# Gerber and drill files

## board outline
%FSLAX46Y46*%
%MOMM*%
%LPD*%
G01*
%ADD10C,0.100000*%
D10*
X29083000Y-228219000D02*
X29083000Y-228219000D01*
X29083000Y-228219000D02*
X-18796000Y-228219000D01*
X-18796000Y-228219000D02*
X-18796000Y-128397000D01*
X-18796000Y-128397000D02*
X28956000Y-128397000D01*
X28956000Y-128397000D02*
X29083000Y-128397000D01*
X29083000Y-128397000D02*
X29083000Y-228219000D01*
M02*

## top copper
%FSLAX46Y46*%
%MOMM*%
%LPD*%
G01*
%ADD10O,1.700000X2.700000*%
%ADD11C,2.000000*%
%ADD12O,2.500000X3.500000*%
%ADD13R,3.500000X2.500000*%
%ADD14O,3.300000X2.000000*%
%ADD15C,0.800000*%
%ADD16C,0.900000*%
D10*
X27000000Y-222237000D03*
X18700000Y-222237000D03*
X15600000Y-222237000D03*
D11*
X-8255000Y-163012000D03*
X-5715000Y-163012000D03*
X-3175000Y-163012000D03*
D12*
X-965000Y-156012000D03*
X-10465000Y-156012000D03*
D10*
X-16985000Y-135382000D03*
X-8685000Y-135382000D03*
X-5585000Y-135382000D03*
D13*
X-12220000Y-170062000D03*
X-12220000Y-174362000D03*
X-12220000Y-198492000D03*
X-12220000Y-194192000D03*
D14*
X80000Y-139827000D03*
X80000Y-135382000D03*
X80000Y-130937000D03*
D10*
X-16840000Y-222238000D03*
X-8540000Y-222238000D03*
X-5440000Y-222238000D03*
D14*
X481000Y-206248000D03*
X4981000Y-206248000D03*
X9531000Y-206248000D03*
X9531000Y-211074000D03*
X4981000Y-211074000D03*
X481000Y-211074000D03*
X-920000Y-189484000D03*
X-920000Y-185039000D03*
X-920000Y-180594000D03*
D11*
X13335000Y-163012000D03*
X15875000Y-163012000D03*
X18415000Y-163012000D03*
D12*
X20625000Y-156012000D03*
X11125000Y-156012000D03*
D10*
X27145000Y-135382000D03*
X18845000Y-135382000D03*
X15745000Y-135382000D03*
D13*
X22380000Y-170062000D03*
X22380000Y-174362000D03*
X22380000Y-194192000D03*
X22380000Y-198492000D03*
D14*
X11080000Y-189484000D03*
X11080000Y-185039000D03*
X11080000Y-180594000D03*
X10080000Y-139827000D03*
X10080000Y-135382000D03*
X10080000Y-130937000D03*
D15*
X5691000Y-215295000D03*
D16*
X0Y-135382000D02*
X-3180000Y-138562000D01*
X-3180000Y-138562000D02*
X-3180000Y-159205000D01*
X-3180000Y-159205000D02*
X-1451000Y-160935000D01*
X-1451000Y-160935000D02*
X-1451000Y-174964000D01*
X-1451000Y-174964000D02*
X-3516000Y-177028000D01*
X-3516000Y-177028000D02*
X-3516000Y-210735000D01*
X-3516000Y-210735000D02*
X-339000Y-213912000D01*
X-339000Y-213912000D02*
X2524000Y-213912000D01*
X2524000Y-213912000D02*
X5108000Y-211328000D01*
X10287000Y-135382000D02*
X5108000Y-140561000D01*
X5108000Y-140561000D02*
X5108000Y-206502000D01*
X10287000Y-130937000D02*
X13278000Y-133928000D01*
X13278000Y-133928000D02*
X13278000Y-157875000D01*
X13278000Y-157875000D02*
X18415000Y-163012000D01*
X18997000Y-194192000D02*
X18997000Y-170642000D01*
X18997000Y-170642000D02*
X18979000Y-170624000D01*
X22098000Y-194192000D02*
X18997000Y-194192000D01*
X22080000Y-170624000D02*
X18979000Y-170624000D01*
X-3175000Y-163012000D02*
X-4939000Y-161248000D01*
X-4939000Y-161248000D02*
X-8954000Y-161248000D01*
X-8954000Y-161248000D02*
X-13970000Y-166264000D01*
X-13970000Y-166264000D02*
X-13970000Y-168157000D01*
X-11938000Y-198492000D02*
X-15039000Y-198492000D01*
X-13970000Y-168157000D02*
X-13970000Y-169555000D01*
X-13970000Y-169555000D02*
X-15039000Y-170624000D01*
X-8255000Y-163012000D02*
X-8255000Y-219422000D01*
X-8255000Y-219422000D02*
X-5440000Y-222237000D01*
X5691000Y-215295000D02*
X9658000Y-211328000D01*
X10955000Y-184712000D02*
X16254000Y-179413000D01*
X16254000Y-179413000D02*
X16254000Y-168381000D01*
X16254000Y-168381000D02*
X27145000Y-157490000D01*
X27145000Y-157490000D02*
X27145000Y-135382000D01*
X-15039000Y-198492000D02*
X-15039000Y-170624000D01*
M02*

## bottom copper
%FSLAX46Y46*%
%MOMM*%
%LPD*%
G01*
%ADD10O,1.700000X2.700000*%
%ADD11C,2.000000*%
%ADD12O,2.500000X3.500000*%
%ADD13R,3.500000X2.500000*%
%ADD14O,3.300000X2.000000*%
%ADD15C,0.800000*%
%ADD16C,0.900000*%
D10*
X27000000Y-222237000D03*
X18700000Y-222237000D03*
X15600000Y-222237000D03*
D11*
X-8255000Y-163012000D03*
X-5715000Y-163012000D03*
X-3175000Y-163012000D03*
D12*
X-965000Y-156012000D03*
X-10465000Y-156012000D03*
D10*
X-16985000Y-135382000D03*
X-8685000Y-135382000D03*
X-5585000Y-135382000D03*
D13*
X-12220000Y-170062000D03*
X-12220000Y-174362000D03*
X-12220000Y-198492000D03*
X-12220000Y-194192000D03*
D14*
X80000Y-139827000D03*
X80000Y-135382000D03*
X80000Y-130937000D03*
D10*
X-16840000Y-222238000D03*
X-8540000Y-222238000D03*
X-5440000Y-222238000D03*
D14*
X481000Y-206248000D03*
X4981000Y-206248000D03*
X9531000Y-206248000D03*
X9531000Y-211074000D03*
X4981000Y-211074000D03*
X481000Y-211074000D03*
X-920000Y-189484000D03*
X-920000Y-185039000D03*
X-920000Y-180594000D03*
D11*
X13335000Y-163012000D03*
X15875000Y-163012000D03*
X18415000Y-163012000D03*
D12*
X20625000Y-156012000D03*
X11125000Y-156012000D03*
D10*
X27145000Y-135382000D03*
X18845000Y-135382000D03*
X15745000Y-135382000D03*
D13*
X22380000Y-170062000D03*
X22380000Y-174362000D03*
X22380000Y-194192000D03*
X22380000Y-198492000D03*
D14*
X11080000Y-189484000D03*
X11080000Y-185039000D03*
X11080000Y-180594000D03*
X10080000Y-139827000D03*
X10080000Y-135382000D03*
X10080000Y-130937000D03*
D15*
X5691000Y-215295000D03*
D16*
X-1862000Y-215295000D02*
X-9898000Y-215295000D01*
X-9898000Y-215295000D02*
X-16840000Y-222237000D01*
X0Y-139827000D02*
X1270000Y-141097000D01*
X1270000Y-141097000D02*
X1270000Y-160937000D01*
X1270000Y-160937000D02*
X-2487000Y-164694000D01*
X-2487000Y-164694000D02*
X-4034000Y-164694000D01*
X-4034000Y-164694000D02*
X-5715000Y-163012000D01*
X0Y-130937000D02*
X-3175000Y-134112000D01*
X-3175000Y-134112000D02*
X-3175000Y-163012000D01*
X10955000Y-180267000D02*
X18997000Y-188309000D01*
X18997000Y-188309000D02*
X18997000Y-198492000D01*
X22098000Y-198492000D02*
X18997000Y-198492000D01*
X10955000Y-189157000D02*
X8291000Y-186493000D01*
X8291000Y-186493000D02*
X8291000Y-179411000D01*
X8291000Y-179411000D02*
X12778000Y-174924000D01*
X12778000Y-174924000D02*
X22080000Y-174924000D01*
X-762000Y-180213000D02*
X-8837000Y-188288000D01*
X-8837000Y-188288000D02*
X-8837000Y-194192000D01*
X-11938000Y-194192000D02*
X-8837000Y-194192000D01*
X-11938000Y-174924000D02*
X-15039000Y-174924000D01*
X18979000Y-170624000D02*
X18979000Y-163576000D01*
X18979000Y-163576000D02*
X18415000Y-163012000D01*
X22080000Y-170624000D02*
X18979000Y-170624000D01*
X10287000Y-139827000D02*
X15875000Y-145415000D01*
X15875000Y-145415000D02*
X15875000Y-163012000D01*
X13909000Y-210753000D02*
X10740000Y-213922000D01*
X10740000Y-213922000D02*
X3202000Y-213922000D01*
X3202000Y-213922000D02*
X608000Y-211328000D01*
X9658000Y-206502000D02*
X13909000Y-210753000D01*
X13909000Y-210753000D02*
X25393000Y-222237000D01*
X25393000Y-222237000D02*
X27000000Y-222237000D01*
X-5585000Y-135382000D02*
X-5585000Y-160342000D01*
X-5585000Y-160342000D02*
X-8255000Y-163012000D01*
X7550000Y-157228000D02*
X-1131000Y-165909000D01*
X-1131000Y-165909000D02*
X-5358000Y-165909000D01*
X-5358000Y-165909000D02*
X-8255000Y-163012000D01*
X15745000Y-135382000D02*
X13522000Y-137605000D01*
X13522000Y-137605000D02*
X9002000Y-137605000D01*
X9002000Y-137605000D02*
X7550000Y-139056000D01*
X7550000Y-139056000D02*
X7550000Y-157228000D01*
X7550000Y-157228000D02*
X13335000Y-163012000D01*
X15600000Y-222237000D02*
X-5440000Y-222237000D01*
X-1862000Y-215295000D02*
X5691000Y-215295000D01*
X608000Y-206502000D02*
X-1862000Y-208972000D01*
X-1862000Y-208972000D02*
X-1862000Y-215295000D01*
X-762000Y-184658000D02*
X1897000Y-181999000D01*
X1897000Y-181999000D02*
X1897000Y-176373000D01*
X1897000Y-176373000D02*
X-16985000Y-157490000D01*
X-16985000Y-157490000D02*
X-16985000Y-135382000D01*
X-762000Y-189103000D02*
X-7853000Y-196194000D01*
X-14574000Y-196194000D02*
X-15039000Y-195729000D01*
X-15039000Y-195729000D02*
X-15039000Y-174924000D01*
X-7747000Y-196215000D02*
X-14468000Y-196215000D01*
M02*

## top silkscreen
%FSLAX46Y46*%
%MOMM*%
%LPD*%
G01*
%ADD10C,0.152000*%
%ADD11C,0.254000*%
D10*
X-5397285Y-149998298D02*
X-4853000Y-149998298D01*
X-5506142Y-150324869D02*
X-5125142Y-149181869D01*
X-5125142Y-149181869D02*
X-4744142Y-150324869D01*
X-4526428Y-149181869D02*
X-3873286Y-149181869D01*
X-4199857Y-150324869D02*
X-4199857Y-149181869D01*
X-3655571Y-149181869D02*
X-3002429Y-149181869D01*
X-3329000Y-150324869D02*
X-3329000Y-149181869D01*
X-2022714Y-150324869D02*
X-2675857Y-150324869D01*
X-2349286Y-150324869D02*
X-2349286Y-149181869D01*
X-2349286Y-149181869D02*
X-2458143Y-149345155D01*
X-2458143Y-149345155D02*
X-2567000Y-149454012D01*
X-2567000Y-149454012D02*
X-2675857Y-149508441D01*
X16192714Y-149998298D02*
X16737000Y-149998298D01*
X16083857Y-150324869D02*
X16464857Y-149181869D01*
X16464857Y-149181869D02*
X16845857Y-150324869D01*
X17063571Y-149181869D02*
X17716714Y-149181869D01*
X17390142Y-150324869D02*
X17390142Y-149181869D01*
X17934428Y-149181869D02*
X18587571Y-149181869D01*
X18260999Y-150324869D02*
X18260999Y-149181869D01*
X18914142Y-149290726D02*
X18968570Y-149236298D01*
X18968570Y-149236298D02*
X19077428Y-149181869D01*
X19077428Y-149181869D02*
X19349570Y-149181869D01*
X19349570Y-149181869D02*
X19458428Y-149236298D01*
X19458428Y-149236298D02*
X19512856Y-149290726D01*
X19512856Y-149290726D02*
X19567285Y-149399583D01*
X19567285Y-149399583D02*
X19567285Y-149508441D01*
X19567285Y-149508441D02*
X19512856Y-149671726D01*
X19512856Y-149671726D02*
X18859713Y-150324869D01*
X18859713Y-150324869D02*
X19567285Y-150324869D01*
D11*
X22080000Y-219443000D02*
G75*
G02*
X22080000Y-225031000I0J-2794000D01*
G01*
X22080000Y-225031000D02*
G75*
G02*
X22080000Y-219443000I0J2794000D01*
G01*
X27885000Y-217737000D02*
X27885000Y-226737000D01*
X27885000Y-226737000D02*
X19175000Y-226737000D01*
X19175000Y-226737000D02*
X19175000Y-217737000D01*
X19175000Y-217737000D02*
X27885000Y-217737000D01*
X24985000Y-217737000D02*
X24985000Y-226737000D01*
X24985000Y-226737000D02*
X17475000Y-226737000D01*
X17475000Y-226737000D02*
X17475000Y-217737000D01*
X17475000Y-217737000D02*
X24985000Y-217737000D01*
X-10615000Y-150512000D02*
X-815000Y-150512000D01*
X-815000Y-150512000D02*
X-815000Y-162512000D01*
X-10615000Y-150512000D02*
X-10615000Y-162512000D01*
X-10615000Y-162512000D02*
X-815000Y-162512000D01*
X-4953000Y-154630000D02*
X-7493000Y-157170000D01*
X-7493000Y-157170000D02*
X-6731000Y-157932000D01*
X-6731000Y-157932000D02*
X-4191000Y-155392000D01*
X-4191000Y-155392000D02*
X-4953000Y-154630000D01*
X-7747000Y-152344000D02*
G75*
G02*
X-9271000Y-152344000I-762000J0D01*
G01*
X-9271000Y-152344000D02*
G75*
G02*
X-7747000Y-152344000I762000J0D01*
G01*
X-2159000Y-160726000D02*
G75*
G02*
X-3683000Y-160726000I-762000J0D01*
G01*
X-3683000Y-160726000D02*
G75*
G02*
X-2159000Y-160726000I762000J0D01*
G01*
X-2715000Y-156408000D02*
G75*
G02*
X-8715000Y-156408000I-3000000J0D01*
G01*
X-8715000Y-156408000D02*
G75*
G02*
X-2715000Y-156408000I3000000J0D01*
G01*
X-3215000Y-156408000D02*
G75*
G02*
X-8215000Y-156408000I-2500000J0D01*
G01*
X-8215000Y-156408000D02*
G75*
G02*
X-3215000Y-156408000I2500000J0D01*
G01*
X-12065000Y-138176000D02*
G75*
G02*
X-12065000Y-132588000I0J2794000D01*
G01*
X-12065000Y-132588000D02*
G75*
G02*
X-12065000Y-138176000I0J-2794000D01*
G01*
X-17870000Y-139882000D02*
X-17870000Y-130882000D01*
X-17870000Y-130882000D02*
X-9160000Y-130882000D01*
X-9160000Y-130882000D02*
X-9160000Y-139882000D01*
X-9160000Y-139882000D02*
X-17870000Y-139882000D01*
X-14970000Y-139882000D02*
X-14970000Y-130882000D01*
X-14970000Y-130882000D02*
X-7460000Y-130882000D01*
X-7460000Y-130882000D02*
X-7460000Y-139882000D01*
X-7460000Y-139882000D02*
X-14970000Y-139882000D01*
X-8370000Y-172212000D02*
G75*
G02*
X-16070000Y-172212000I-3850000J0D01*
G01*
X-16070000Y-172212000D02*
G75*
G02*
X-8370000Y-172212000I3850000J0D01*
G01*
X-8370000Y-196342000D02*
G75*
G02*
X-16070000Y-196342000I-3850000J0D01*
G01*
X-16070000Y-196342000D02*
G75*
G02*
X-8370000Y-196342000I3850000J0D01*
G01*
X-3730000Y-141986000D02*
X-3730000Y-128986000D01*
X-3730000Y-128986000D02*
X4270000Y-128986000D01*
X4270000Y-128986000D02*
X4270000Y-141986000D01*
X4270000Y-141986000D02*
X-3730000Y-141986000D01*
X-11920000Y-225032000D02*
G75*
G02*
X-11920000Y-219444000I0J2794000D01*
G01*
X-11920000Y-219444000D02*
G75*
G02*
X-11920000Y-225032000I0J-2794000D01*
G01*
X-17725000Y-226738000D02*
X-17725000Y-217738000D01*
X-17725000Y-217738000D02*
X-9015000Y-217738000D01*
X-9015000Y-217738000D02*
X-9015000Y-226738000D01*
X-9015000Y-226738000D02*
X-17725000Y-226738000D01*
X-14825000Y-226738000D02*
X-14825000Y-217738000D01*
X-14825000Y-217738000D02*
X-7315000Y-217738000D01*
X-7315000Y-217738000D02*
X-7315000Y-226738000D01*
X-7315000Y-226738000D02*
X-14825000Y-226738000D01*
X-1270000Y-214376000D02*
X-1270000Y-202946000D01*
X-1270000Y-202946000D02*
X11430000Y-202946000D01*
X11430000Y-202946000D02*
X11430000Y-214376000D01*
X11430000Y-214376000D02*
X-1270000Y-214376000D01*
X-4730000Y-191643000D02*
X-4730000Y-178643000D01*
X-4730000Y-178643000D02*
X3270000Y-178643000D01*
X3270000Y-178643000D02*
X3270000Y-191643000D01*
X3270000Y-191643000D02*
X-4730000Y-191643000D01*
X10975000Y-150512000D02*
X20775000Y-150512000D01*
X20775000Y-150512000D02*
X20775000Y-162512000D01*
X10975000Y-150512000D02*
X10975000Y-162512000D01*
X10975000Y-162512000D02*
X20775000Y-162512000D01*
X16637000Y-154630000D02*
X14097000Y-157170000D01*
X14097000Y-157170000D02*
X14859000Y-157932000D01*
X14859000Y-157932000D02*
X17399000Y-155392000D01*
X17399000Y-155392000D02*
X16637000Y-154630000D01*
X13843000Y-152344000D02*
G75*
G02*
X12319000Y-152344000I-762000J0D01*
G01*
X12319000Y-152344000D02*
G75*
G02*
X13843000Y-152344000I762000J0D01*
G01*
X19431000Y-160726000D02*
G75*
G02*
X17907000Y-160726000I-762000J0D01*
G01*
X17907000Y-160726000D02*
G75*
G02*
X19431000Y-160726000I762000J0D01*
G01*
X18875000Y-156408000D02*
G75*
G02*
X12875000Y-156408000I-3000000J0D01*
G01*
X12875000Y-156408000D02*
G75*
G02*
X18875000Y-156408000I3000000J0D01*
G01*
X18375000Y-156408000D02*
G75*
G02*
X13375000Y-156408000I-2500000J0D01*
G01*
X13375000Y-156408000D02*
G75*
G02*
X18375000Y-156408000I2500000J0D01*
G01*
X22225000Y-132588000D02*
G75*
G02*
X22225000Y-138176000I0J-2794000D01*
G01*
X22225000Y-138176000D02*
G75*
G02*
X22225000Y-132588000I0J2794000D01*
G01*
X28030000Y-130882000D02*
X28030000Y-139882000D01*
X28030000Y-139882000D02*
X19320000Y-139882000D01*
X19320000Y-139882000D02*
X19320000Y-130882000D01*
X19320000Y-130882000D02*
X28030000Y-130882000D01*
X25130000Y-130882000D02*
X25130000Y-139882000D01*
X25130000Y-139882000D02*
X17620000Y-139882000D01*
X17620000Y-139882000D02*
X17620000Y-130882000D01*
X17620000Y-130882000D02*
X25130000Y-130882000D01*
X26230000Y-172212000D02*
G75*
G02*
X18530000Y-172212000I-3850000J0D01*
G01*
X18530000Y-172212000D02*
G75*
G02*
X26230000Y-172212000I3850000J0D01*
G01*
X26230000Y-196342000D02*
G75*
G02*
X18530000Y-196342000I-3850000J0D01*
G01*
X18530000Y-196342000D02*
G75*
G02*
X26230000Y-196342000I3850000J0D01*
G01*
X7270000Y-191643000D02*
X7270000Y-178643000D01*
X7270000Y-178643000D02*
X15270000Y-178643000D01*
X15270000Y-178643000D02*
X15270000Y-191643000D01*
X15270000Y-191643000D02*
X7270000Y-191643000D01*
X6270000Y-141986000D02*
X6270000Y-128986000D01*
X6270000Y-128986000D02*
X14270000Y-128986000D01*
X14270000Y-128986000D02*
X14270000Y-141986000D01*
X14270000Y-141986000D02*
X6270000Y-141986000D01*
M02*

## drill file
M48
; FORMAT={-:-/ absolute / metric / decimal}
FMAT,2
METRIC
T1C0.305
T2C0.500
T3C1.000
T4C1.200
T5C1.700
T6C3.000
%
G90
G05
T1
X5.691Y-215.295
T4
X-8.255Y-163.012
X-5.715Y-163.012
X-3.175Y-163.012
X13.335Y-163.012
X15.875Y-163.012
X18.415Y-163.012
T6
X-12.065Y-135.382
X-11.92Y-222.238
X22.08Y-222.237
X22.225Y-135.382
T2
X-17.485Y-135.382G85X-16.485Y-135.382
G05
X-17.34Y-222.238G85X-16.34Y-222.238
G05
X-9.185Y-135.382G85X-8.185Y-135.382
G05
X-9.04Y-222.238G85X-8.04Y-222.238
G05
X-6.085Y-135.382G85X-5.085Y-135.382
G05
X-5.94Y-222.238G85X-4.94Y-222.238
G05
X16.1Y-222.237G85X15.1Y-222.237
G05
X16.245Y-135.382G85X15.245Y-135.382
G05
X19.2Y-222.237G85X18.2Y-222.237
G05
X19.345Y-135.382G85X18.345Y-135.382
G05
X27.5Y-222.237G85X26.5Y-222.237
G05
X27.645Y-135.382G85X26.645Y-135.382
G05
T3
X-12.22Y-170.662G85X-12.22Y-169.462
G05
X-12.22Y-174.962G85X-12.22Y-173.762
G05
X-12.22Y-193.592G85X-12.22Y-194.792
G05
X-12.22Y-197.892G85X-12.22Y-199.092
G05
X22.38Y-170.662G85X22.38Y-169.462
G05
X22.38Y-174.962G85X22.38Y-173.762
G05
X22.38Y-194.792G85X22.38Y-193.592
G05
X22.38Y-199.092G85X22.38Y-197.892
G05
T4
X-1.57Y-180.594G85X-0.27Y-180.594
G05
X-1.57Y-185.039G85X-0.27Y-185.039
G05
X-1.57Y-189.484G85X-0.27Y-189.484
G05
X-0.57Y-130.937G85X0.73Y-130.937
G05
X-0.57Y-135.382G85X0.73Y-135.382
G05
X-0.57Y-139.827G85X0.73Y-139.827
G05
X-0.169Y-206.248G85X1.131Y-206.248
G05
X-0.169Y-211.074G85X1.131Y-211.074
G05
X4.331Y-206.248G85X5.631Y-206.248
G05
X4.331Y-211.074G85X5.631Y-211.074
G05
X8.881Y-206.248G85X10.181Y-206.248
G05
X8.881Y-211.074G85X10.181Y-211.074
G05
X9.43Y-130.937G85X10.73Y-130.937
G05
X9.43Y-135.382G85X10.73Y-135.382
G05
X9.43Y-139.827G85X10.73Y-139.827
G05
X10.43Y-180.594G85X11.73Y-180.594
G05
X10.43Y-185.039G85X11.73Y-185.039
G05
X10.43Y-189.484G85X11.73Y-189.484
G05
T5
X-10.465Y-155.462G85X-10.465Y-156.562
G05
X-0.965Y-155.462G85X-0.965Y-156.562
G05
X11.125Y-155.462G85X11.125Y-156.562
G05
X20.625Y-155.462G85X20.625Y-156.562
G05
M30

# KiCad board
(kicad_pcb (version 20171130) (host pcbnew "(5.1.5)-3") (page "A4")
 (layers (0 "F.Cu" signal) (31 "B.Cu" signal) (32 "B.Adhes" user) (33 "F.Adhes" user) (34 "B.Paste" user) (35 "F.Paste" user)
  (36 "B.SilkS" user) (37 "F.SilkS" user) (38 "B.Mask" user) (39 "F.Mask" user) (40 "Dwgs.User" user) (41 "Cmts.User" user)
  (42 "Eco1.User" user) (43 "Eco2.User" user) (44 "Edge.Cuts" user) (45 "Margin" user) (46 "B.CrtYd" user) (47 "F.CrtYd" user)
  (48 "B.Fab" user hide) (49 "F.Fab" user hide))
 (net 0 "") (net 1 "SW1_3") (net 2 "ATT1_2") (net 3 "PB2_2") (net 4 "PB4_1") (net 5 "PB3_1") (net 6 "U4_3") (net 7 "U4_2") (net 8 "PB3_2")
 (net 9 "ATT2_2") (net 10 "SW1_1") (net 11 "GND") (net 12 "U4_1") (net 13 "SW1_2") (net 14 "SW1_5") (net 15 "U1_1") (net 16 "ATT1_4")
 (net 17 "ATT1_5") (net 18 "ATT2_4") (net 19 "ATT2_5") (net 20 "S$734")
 (segment (start -1.862 215.295) (end -9.898 215.295) (width 0.9) (layer "B.Cu") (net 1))
 (segment (start -9.898 215.295) (end -16.84 222.237) (width 0.9) (layer "B.Cu") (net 1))
 (segment (start 0 139.827) (end 1.27 141.097) (width 0.9) (layer "B.Cu") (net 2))
 (segment (start 1.27 141.097) (end 1.27 160.937) (width 0.9) (layer "B.Cu") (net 2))
 (segment (start 1.27 160.937) (end -2.487 164.694) (width 0.9) (layer "B.Cu") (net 2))
 (segment (start -2.487 164.694) (end -4.034 164.694) (width 0.9) (layer "B.Cu") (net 2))
 (segment (start -4.034 164.694) (end -5.715 163.012) (width 0.9) (layer "B.Cu") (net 2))
 (segment (start 0 130.937) (end -3.175 134.112) (width 0.9) (layer "B.Cu") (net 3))
 (segment (start -3.175 134.112) (end -3.175 163.012) (width 0.9) (layer "B.Cu") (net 3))
 (segment (start 10.955 180.267) (end 18.997 188.309) (width 0.9) (layer "B.Cu") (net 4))
 (segment (start 18.997 188.309) (end 18.997 198.492) (width 0.9) (layer "B.Cu") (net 4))
 (segment (start 22.098 198.492) (end 18.997 198.492) (width 0.9) (layer "B.Cu") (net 4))
 (segment (start 10.955 189.157) (end 8.291 186.493) (width 0.9) (layer "B.Cu") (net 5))
 (segment (start 8.291 186.493) (end 8.291 179.411) (width 0.9) (layer "B.Cu") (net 5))
 (segment (start 8.291 179.411) (end 12.778 174.924) (width 0.9) (layer "B.Cu") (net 5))
 (segment (start 12.778 174.924) (end 22.08 174.924) (width 0.9) (layer "B.Cu") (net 5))
 (segment (start -0.762 180.213) (end -8.837 188.288) (width 0.9) (layer "B.Cu") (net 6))
 (segment (start -8.837 188.288) (end -8.837 194.192) (width 0.9) (layer "B.Cu") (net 6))
 (segment (start -11.938 194.192) (end -8.837 194.192) (width 0.9) (layer "B.Cu") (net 6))
 (segment (start -11.938 174.924) (end -15.039 174.924) (width 0.9) (layer "B.Cu") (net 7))
 (segment (start 18.979 170.624) (end 18.979 163.576) (width 0.9) (layer "B.Cu") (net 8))
 (segment (start 18.979 163.576) (end 18.415 163.012) (width 0.9) (layer "B.Cu") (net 8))
 (segment (start 22.08 170.624) (end 18.979 170.624) (width 0.9) (layer "B.Cu") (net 8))
 (segment (start 10.287 139.827) (end 15.875 145.415) (width 0.9) (layer "B.Cu") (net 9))
 (segment (start 15.875 145.415) (end 15.875 163.012) (width 0.9) (layer "B.Cu") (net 9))
 (segment (start 13.909 210.753) (end 10.74 213.922) (width 0.9) (layer "B.Cu") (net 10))
 (segment (start 10.74 213.922) (end 3.202 213.922) (width 0.9) (layer "B.Cu") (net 10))
 (segment (start 3.202 213.922) (end 0.608 211.328) (width 0.9) (layer "B.Cu") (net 10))
 (segment (start 9.658 206.502) (end 13.909 210.753) (width 0.9) (layer "B.Cu") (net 10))
 (segment (start 13.909 210.753) (end 25.393 222.237) (width 0.9) (layer "B.Cu") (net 10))
 (segment (start 25.393 222.237) (end 27 222.237) (width 0.9) (layer "B.Cu") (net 10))
 (segment (start -5.585 135.382) (end -5.585 160.342) (width 0.9) (layer "B.Cu") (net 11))
 (segment (start -5.585 160.342) (end -8.255 163.012) (width 0.9) (layer "B.Cu") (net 11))
 (segment (start 7.55 157.228) (end -1.131 165.909) (width 0.9) (layer "B.Cu") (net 11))
 (segment (start -1.131 165.909) (end -5.358 165.909) (width 0.9) (layer "B.Cu") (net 11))
 (segment (start -5.358 165.909) (end -8.255 163.012) (width 0.9) (layer "B.Cu") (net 11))
 (segment (start 15.745 135.382) (end 13.522 137.605) (width 0.9) (layer "B.Cu") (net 11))
 (segment (start 13.522 137.605) (end 9.002 137.605) (width 0.9) (layer "B.Cu") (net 11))
 (segment (start 9.002 137.605) (end 7.55 139.056) (width 0.9) (layer "B.Cu") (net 11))
 (segment (start 7.55 139.056) (end 7.55 157.228) (width 0.9) (layer "B.Cu") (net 11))
 (segment (start 7.55 157.228) (end 13.335 163.012) (width 0.9) (layer "B.Cu") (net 11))
 (segment (start 15.6 222.237) (end -5.44 222.237) (width 0.9) (layer "B.Cu") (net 11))
 (segment (start -1.862 215.295) (end 5.691 215.295) (width 0.9) (layer "B.Cu") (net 1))
 (segment (start 0.608 206.502) (end -1.862 208.972) (width 0.9) (layer "B.Cu") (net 1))
 (segment (start -1.862 208.972) (end -1.862 215.295) (width 0.9) (layer "B.Cu") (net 1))
 (segment (start -0.762 184.658) (end 1.897 181.999) (width 0.9) (layer "B.Cu") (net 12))
 (segment (start 1.897 181.999) (end 1.897 176.373) (width 0.9) (layer "B.Cu") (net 12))
 (segment (start 1.897 176.373) (end -16.985 157.49) (width 0.9) (layer "B.Cu") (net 12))
 (segment (start -16.985 157.49) (end -16.985 135.382) (width 0.9) (layer "B.Cu") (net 12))
 (segment (start -0.762 189.103) (end -7.853 196.194) (width 0.9) (layer "B.Cu") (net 7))
 (segment (start -14.574 196.194) (end -15.039 195.729) (width 0.9) (layer "B.Cu") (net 7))
 (segment (start -15.039 195.729) (end -15.039 174.924) (width 0.9) (layer "B.Cu") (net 7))
 (segment (start -7.747 196.215) (end -14.468 196.215) (width 0.9) (layer "B.Cu") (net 7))
 (gr_line (start 29.083 228.219) (end 29.083 228.219) (width 0.1) (layer "Edge.Cuts"))
 (gr_line (start 29.083 228.219) (end -18.796 228.219) (width 0.1) (layer "Edge.Cuts"))
 (gr_line (start -18.796 228.219) (end -18.796 128.397) (width 0.1) (layer "Edge.Cuts"))
 (gr_line (start -18.796 128.397) (end 28.956 128.397) (width 0.1) (layer "Edge.Cuts"))
 (gr_line (start 28.956 128.397) (end 29.083 128.397) (width 0.1) (layer "Edge.Cuts"))
 (gr_line (start 29.083 128.397) (end 29.083 228.219) (width 0.1) (layer "Edge.Cuts"))
 (segment (start 0 135.382) (end -3.18 138.562) (width 0.9) (layer "F.Cu") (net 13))
 (segment (start -3.18 138.562) (end -3.18 159.205) (width 0.9) (layer "F.Cu") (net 13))
 (segment (start -3.18 159.205) (end -1.451 160.935) (width 0.9) (layer "F.Cu") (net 13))
 (segment (start -1.451 160.935) (end -1.451 174.964) (width 0.9) (layer "F.Cu") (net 13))
 (segment (start -1.451 174.964) (end -3.516 177.028) (width 0.9) (layer "F.Cu") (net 13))
 (segment (start -3.516 177.028) (end -3.516 210.735) (width 0.9) (layer "F.Cu") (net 13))
 (segment (start -3.516 210.735) (end -0.339 213.912) (width 0.9) (layer "F.Cu") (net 13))
 (segment (start -0.339 213.912) (end 2.524 213.912) (width 0.9) (layer "F.Cu") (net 13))
 (segment (start 2.524 213.912) (end 5.108 211.328) (width 0.9) (layer "F.Cu") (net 13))
 (segment (start 10.287 135.382) (end 5.108 140.561) (width 0.9) (layer "F.Cu") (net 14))
 (segment (start 5.108 140.561) (end 5.108 206.502) (width 0.9) (layer "F.Cu") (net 14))
 (segment (start 10.287 130.937) (end 13.278 133.928) (width 0.9) (layer "F.Cu") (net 8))
 (segment (start 13.278 133.928) (end 13.278 157.875) (width 0.9) (layer "F.Cu") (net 8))
 (segment (start 13.278 157.875) (end 18.415 163.012) (width 0.9) (layer "F.Cu") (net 8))
 (segment (start 18.997 194.192) (end 18.997 170.642) (width 0.9) (layer "F.Cu") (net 8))
 (segment (start 18.997 170.642) (end 18.979 170.624) (width 0.9) (layer "F.Cu") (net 8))
 (segment (start 22.098 194.192) (end 18.997 194.192) (width 0.9) (layer "F.Cu") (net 8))
 (segment (start 22.08 170.624) (end 18.979 170.624) (width 0.9) (layer "F.Cu") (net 8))
 (segment (start -3.175 163.012) (end -4.939 161.248) (width 0.9) (layer "F.Cu") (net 3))
 (segment (start -4.939 161.248) (end -8.954 161.248) (width 0.9) (layer "F.Cu") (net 3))
 (segment (start -8.954 161.248) (end -13.97 166.264) (width 0.9) (layer "F.Cu") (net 3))
 (segment (start -13.97 166.264) (end -13.97 168.157) (width 0.9) (layer "F.Cu") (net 3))
 (segment (start -11.938 198.492) (end -15.039 198.492) (width 0.9) (layer "F.Cu") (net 3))
 (segment (start -13.97 168.157) (end -13.97 169.555) (width 0.9) (layer "F.Cu") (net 3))
 (segment (start -13.97 169.555) (end -15.039 170.624) (width 0.9) (layer "F.Cu") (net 3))
 (segment (start -8.255 163.012) (end -8.255 219.422) (width 0.9) (layer "F.Cu") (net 11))
 (segment (start -8.255 219.422) (end -5.44 222.237) (width 0.9) (layer "F.Cu") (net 11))
 (segment (start 5.691 215.295) (end 9.658 211.328) (width 0.9) (layer "F.Cu") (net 1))
 (segment (start 10.955 184.712) (end 16.254 179.413) (width 0.9) (layer "F.Cu") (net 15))
 (segment (start 16.254 179.413) (end 16.254 168.381) (width 0.9) (layer "F.Cu") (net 15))
 (segment (start 16.254 168.381) (end 27.145 157.49) (width 0.9) (layer "F.Cu") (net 15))
 (segment (start 27.145 157.49) (end 27.145 135.382) (width 0.9) (layer "F.Cu") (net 15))
 (segment (start -15.039 198.492) (end -15.039 170.624) (width 0.9) (layer "F.Cu") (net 3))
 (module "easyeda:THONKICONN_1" (layer "F.Cu") (at 22.08 222.237 -90)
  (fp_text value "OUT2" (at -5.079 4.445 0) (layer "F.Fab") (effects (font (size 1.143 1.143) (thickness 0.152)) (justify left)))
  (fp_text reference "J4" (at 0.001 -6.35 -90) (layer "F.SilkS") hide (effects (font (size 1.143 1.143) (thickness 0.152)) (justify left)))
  (fp_arc (start 0 0) (end -2.794 0) (angle 180) (width 0.254) (layer "F.SilkS"))
  (fp_arc (start 0 0) (end 2.794 0) (angle 180) (width 0.254) (layer "F.SilkS"))
  (fp_line (start -4.5 -5.805) (end 4.5 -5.805) (width 0.254) (layer "F.SilkS"))
  (fp_line (start 4.5 -5.805) (end 4.5 2.905) (width 0.254) (layer "F.SilkS"))
  (fp_line (start 4.5 2.905) (end -4.5 2.905) (width 0.254) (layer "F.SilkS"))
  (fp_line (start -4.5 2.905) (end -4.5 -5.805) (width 0.254) (layer "F.SilkS"))
  (fp_line (start -4.5 -2.905) (end 4.5 -2.905) (width 0.254) (layer "F.SilkS"))
  (fp_line (start 4.5 -2.905) (end 4.5 4.605) (width 0.254) (layer "F.SilkS"))
  (fp_line (start 4.5 4.605) (end -4.5 4.605) (width 0.254) (layer "F.SilkS"))
  (fp_line (start -4.5 4.605) (end -4.5 -2.905) (width 0.254) (layer "F.SilkS"))
  (pad "" np_thru_hole circle (at 0 0) (size 3 3) (drill 3) (layers "*.Cu" "*.Mask"))
  (pad 3 thru_hole oval (at 0 -4.92 -90) (size 2.7 1.7) (layers "*.Cu" "*.Paste" "*.Mask") (drill oval 0.5 1.5) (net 10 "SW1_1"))
  (pad 2 thru_hole oval (at 0 3.38 -90) (size 2.7 1.7) (layers "*.Cu" "*.Paste" "*.Mask") (drill oval 0.5 1.5))
  (pad 1 thru_hole oval (at 0 6.48 -90) (size 2.7 1.7) (layers "*.Cu" "*.Paste" "*.Mask") (drill oval 0.5 1.5) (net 11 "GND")))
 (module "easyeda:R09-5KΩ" (layer "F.Cu") (at -5.715 159.512)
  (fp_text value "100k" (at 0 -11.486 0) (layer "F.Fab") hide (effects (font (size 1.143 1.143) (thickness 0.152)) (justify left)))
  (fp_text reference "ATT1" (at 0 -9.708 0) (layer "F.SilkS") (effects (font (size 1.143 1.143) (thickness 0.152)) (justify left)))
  (fp_line (start -4.9 -9) (end 4.9 -9) (width 0.254) (layer "F.SilkS"))
  (fp_line (start 4.9 -9) (end 4.9 3) (width 0.254) (layer "F.SilkS"))
  (fp_line (start -4.9 -9) (end -4.9 3) (width 0.254) (layer "F.SilkS"))
  (fp_line (start -4.9 3) (end 4.9 3) (width 0.254) (layer "F.SilkS"))
  (fp_line (start 0.762 -4.882) (end -1.778 -2.342) (width 0.254) (layer "F.SilkS"))
  (fp_line (start -1.778 -2.342) (end -1.016 -1.58) (width 0.254) (layer "F.SilkS"))
  (fp_line (start -1.016 -1.58) (end 1.524 -4.12) (width 0.254) (layer "F.SilkS"))
  (fp_line (start 1.524 -4.12) (end 0.762 -4.882) (width 0.254) (layer "F.SilkS"))
  (fp_circle (center -2.794 -7.168) (end -2.032 -7.168) (layer "F.SilkS") (width 0.254))
  (fp_circle (center 2.794 1.214) (end 3.556 1.214) (layer "F.SilkS") (width 0.254))
  (fp_circle (center 0 -3.104) (end 3 -3.104) (layer "F.SilkS") (width 0.254))
  (fp_circle (center 0 -3.104) (end 2.5 -3.104) (layer "F.SilkS") (width 0.254))
  (pad 1 thru_hole circle (at -2.54 3.5 0) (size 2 2) (layers "*.Cu" "*.Paste" "*.Mask") (drill 1.2) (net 11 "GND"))
  (pad 2 thru_hole circle (at 0 3.5 0) (size 2 2) (layers "*.Cu" "*.Paste" "*.Mask") (drill 1.2) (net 2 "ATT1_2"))
  (pad 3 thru_hole circle (at 2.54 3.5 0) (size 2 2) (layers "*.Cu" "*.Paste" "*.Mask") (drill 1.2) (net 3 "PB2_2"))
  (pad 4 thru_hole oval (at 4.75 -3.5 0) (size 2.5 3.5) (layers "*.Cu" "*.Paste" "*.Mask") (drill oval 1.7 2.8) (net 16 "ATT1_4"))
  (pad 5 thru_hole oval (at -4.75 -3.5 0) (size 2.5 3.5) (layers "*.Cu" "*.Paste" "*.Mask") (drill oval 1.7 2.8) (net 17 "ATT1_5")))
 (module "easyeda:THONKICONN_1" (layer "F.Cu") (at -12.065 135.382 90)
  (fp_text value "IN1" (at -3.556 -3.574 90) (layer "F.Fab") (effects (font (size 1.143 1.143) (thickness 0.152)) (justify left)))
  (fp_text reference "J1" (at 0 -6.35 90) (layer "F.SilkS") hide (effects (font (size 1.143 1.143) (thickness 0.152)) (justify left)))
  (fp_arc (start 0 0) (end -2.794 0) (angle 180) (width 0.254) (layer "F.SilkS"))
  (fp_arc (start 0 0) (end 2.794 0) (angle 180) (width 0.254) (layer "F.SilkS"))
  (pad "" np_thru_hole circle (at 0 0) (size 3 3) (drill 3) (layers "*.Cu" "*.Mask"))
  (fp_line (start -4.5 -5.805) (end 4.5 -5.805) (width 0.254) (layer "F.SilkS"))
  (fp_line (start 4.5 -5.805) (end 4.5 2.905) (width 0.254) (layer "F.SilkS"))
  (fp_line (start 4.5 2.905) (end -4.5 2.905) (width 0.254) (layer "F.SilkS"))
  (fp_line (start -4.5 2.905) (end -4.5 -5.805) (width 0.254) (layer "F.SilkS"))
  (fp_line (start -4.5 -2.905) (end 4.5 -2.905) (width 0.254) (layer "F.SilkS"))
  (fp_line (start 4.5 -2.905) (end 4.5 4.605) (width 0.254) (layer "F.SilkS"))
  (fp_line (start 4.5 4.605) (end -4.5 4.605) (width 0.254) (layer "F.SilkS"))
  (fp_line (start -4.5 4.605) (end -4.5 -2.905) (width 0.254) (layer "F.SilkS"))
  (pad 3 thru_hole oval (at 0 -4.92 90) (size 2.7 1.7) (layers "*.Cu" "*.Paste" "*.Mask") (drill oval 0.5 1.5) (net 12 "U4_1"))
  (pad 2 thru_hole oval (at 0 3.38 90) (size 2.7 1.7) (layers "*.Cu" "*.Paste" "*.Mask") (drill oval 0.5 1.5))
  (pad 1 thru_hole oval (at 0 6.48 90) (size 2.7 1.7) (layers "*.Cu" "*.Paste" "*.Mask") (drill oval 0.5 1.5) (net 11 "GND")))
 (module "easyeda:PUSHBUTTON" (layer "F.Cu") (at -12.22 172.212 90)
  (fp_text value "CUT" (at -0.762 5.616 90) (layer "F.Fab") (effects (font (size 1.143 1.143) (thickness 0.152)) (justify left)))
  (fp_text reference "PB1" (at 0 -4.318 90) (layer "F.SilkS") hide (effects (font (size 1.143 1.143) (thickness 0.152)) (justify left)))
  (fp_circle (center 0 0) (end 3.85 0) (layer "F.SilkS") (width 0.254))
  (pad 2 thru_hole rect (at 2.15 0 180) (size 3.5 2.5) (layers "*.Cu" "*.Paste" "*.Mask") (drill oval 1 2.2) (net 3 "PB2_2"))
  (pad 1 thru_hole rect (at -2.15 0 180) (size 3.5 2.5) (layers "*.Cu" "*.Paste" "*.Mask") (drill oval 1 2.2) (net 7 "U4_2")))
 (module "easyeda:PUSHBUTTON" (layer "F.Cu") (at -12.22 196.342 -90)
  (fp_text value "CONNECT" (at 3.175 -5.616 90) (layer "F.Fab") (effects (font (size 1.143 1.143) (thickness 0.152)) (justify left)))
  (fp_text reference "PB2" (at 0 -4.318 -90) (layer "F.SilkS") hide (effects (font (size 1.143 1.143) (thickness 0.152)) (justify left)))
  (fp_circle (center 0 0) (end 3.85 0) (layer "F.SilkS") (width 0.254))
  (pad 2 thru_hole rect (at 2.15 0 0) (size 3.5 2.5) (layers "*.Cu" "*.Paste" "*.Mask") (drill oval 1 2.2) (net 3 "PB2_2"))
  (pad 1 thru_hole rect (at -2.15 0 0) (size 3.5 2.5) (layers "*.Cu" "*.Paste" "*.Mask") (drill oval 1 2.2) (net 6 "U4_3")))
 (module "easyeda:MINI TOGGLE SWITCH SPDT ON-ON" (layer "F.Cu") (at 0.08 135.382 90)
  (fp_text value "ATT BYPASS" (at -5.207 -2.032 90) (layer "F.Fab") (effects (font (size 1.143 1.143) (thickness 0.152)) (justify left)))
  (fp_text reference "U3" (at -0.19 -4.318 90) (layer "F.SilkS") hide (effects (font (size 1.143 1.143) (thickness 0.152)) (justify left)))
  (fp_line (start -6.604 -3.81) (end 6.396 -3.81) (width 0.254) (layer "F.SilkS") (status 40000))
  (fp_line (start 6.396 -3.81) (end 6.396 4.19) (width 0.254) (layer "F.SilkS") (status 40000))
  (fp_line (start 6.396 4.19) (end -6.604 4.19) (width 0.254) (layer "F.SilkS") (status 40000))
  (fp_line (start -6.604 4.19) (end -6.604 -3.81) (width 0.254) (layer "F.SilkS") (status 40000))
  (pad 2 thru_hole oval (at -4.445 0 90) (size 2 3.3) (layers "*.Cu" "*.Paste" "*.Mask") (drill oval 1.2 2.5) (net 2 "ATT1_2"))
  (pad 1 thru_hole oval (at 0 0 90) (size 2 3.3) (layers "*.Cu" "*.Paste" "*.Mask") (drill oval 1.2 2.5) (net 13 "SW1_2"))
  (pad 3 thru_hole oval (at 4.445 0 90) (size 2 3.3) (layers "*.Cu" "*.Paste" "*.Mask") (drill oval 1.2 2.5) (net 3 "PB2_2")))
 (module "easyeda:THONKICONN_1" (layer "F.Cu") (at -11.92 222.238 90)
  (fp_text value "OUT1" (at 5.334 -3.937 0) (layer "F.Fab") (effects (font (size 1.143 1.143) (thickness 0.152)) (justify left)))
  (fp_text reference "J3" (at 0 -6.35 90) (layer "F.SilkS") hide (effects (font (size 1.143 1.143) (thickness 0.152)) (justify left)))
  (fp_arc (start 0 0) (end -2.794 0) (angle 180) (width 0.254) (layer "F.SilkS"))
  (fp_arc (start 0 0) (end 2.794 0) (angle 180) (width 0.254) (layer "F.SilkS"))
  (fp_line (start -4.5 -5.805) (end 4.5 -5.805) (width 0.254) (layer "F.SilkS"))
  (fp_line (start 4.5 -5.805) (end 4.5 2.905) (width 0.254) (layer "F.SilkS"))
  (fp_line (start 4.5 2.905) (end -4.5 2.905) (width 0.254) (layer "F.SilkS"))
  (fp_line (start -4.5 2.905) (end -4.5 -5.805) (width 0.254) (layer "F.SilkS"))
  (fp_line (start -4.5 -2.905) (end 4.5 -2.905) (width 0.254) (layer "F.SilkS"))
  (fp_line (start 4.5 -2.905) (end 4.5 4.605) (width 0.254) (layer "F.SilkS"))
  (fp_line (start 4.5 4.605) (end -4.5 4.605) (width 0.254) (layer "F.SilkS"))
  (fp_line (start -4.5 4.605) (end -4.5 -2.905) (width 0.254) (layer "F.SilkS"))
  (pad "" np_thru_hole circle (at 0 0) (size 3 3) (drill 3) (layers "*.Cu" "*.Mask"))
  (pad 3 thru_hole oval (at 0 -4.92 90) (size 2.7 1.7) (layers "*.Cu" "*.Paste" "*.Mask") (drill oval 0.5 1.5) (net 1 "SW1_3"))
  (pad 2 thru_hole oval (at 0 3.38 90) (size 2.7 1.7) (layers "*.Cu" "*.Paste" "*.Mask") (drill oval 0.5 1.5))
  (pad 1 thru_hole oval (at 0 6.48 90) (size 2.7 1.7) (layers "*.Cu" "*.Paste" "*.Mask") (drill oval 0.5 1.5) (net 11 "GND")))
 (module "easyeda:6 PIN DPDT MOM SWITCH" (layer "F.Cu") (at 11.43 214.376 90)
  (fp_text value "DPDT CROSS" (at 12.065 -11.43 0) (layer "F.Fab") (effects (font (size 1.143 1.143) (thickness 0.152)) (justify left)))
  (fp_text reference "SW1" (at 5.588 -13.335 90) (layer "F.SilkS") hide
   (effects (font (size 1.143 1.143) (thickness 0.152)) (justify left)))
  (fp_line (start 0 -12.7) (end 11.43 -12.7) (width 0.254) (layer "F.SilkS"))
  (fp_line (start 11.43 -12.7) (end 11.43 0) (width 0.254) (layer "F.SilkS"))
  (fp_line (start 11.43 0) (end 0 0) (width 0.254) (layer "F.SilkS"))
  (fp_line (start 0 0) (end 0 -12.7) (width 0.254) (layer "F.SilkS"))
  (pad 4 thru_hole oval (at 8.128 -10.949 90) (size 2 3.3) (layers "*.Cu" "*.Paste" "*.Mask") (drill oval 1.2 2.5) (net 1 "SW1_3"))
  (pad 5 thru_hole oval (at 8.128 -6.449 90) (size 2 3.3) (layers "*.Cu" "*.Paste" "*.Mask") (drill oval 1.2 2.5) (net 14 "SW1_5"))
  (pad 6 thru_hole oval (at 8.128 -1.899 90) (size 2 3.3) (layers "*.Cu" "*.Paste" "*.Mask") (drill oval 1.2 2.5) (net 10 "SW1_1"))
  (pad 3 thru_hole oval (at 3.302 -1.899 90) (size 2 3.3) (layers "*.Cu" "*.Paste" "*.Mask") (drill oval 1.2 2.5) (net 1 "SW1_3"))
  (pad 2 thru_hole oval (at 3.302 -6.449 90) (size 2 3.3) (layers "*.Cu" "*.Paste" "*.Mask") (drill oval 1.2 2.5) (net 13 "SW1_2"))
  (pad 1 thru_hole oval (at 3.302 -10.949 90) (size 2 3.3) (layers "*.Cu" "*.Paste" "*.Mask") (drill oval 1.2 2.5) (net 10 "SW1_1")))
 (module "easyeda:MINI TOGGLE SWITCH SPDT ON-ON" (layer "F.Cu") (at -0.92 185.039 90)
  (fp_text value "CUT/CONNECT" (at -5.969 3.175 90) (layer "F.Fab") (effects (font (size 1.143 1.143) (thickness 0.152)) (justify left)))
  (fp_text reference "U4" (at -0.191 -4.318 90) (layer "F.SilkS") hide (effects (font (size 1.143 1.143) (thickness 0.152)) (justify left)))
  (fp_line (start -6.604 -3.81) (end 6.396 -3.81) (width 0.254) (layer "F.SilkS") (status 40000))
  (fp_line (start 6.396 -3.81) (end 6.396 4.19) (width 0.254) (layer "F.SilkS") (status 40000))
  (fp_line (start 6.396 4.19) (end -6.604 4.19) (width 0.254) (layer "F.SilkS") (status 40000))
  (fp_line (start -6.604 4.19) (end -6.604 -3.81) (width 0.254) (layer "F.SilkS") (status 40000))
  (pad 2 thru_hole oval (at -4.445 0 90) (size 2 3.3) (layers "*.Cu" "*.Paste" "*.Mask") (drill oval 1.2 2.5) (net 7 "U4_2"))
  (pad 1 thru_hole oval (at 0 0 90) (size 2 3.3) (layers "*.Cu" "*.Paste" "*.Mask") (drill oval 1.2 2.5) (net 12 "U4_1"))
  (pad 3 thru_hole oval (at 4.445 0 90) (size 2 3.3) (layers "*.Cu" "*.Paste" "*.Mask") (drill oval 1.2 2.5) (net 6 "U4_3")))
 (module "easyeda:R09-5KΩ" (layer "F.Cu") (at 15.875 159.512)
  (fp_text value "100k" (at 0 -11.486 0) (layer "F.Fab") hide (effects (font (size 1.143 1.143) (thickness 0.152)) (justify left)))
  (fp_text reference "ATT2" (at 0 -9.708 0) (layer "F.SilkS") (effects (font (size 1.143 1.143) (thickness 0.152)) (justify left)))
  (fp_line (start -4.9 -9) (end 4.9 -9) (width 0.254) (layer "F.SilkS"))
  (fp_line (start 4.9 -9) (end 4.9 3) (width 0.254) (layer "F.SilkS"))
  (fp_line (start -4.9 -9) (end -4.9 3) (width 0.254) (layer "F.SilkS"))
  (fp_line (start -4.9 3) (end 4.9 3) (width 0.254) (layer "F.SilkS"))
  (fp_line (start 0.762 -4.882) (end -1.778 -2.342) (width 0.254) (layer "F.SilkS"))
  (fp_line (start -1.778 -2.342) (end -1.016 -1.58) (width 0.254) (layer "F.SilkS"))
  (fp_line (start -1.016 -1.58) (end 1.524 -4.12) (width 0.254) (layer "F.SilkS"))
  (fp_line (start 1.524 -4.12) (end 0.762 -4.882) (width 0.254) (layer "F.SilkS"))
  (fp_circle (center -2.794 -7.168) (end -2.032 -7.168) (layer "F.SilkS") (width 0.254))
  (fp_circle (center 2.794 1.214) (end 3.556 1.214) (layer "F.SilkS") (width 0.254))
  (fp_circle (center 0 -3.104) (end 3 -3.104) (layer "F.SilkS") (width 0.254))
  (fp_circle (center 0 -3.104) (end 2.5 -3.104) (layer "F.SilkS") (width 0.254))
  (pad 1 thru_hole circle (at -2.54 3.5 0) (size 2 2) (layers "*.Cu" "*.Paste" "*.Mask") (drill 1.2) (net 11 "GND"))
  (pad 2 thru_hole circle (at 0 3.5 0) (size 2 2) (layers "*.Cu" "*.Paste" "*.Mask") (drill 1.2) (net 9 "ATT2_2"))
  (pad 3 thru_hole circle (at 2.54 3.5 0) (size 2 2) (layers "*.Cu" "*.Paste" "*.Mask") (drill 1.2) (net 8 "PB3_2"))
  (pad 4 thru_hole oval (at 4.75 -3.5 0) (size 2.5 3.5) (layers "*.Cu" "*.Paste" "*.Mask") (drill oval 1.7 2.8) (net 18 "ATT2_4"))
  (pad 5 thru_hole oval (at -4.75 -3.5 0) (size 2.5 3.5) (layers "*.Cu" "*.Paste" "*.Mask") (drill oval 1.7 2.8) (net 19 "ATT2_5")))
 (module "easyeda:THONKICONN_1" (layer "F.Cu") (at 22.225 135.382 -90)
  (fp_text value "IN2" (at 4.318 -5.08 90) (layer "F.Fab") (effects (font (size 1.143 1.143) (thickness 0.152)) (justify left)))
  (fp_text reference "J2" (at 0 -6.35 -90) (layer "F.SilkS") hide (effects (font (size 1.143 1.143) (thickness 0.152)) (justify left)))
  (fp_arc (start 0 0) (end -2.794 0) (angle 180) (width 0.254) (layer "F.SilkS"))
  (fp_arc (start 0 0) (end 2.794 0) (angle 180) (width 0.254) (layer "F.SilkS"))
  (pad "" np_thru_hole circle (at 0 0) (size 3 3) (drill 3) (layers "*.Cu" "*.Mask"))
  (fp_line (start -4.5 -5.805) (end 4.5 -5.805) (width 0.254) (layer "F.SilkS"))
  (fp_line (start 4.5 -5.805) (end 4.5 2.905) (width 0.254) (layer "F.SilkS"))
  (fp_line (start 4.5 2.905) (end -4.5 2.905) (width 0.254) (layer "F.SilkS"))
  (fp_line (start -4.5 2.905) (end -4.5 -5.805) (width 0.254) (layer "F.SilkS"))
  (fp_line (start -4.5 -2.905) (end 4.5 -2.905) (width 0.254) (layer "F.SilkS"))
  (fp_line (start 4.5 -2.905) (end 4.5 4.605) (width 0.254) (layer "F.SilkS"))
  (fp_line (start 4.5 4.605) (end -4.5 4.605) (width 0.254) (layer "F.SilkS"))
  (fp_line (start -4.5 4.605) (end -4.5 -2.905) (width 0.254) (layer "F.SilkS"))
  (pad 3 thru_hole oval (at 0 -4.92 -90) (size 2.7 1.7) (layers "*.Cu" "*.Paste" "*.Mask") (drill oval 0.5 1.5) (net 15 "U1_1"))
  (pad 2 thru_hole oval (at 0 3.38 -90) (size 2.7 1.7) (layers "*.Cu" "*.Paste" "*.Mask") (drill oval 0.5 1.5))
  (pad 1 thru_hole oval (at 0 6.48 -90) (size 2.7 1.7) (layers "*.Cu" "*.Paste" "*.Mask") (drill oval 0.5 1.5) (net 11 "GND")))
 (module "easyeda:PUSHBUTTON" (layer "F.Cu") (at 22.38 172.212 90)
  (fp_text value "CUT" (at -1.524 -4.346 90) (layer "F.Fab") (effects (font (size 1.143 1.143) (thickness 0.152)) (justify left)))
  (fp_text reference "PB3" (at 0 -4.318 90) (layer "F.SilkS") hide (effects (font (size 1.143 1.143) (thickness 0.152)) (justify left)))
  (fp_circle (center 0 0) (end 3.85 0) (layer "F.SilkS") (width 0.254))
  (pad 2 thru_hole rect (at 2.15 0 180) (size 3.5 2.5) (layers "*.Cu" "*.Paste" "*.Mask") (drill oval 1 2.2) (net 8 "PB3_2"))
  (pad 1 thru_hole rect (at -2.15 0 180) (size 3.5 2.5) (layers "*.Cu" "*.Paste" "*.Mask") (drill oval 1 2.2) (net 5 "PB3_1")))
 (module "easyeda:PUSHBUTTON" (layer "F.Cu") (at 22.38 196.342 90)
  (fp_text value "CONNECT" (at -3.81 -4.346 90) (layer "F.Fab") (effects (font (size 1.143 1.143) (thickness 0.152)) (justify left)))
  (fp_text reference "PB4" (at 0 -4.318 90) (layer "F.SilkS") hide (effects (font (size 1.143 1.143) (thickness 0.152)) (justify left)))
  (fp_circle (center 0 0) (end 3.85 0) (layer "F.SilkS") (width 0.254))
  (pad 2 thru_hole rect (at 2.15 0 180) (size 3.5 2.5) (layers "*.Cu" "*.Paste" "*.Mask") (drill oval 1 2.2) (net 8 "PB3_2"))
  (pad 1 thru_hole rect (at -2.15 0 180) (size 3.5 2.5) (layers "*.Cu" "*.Paste" "*.Mask") (drill oval 1 2.2) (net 4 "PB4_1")))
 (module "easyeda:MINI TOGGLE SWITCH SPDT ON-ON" (layer "F.Cu") (at 11.08 185.039 90)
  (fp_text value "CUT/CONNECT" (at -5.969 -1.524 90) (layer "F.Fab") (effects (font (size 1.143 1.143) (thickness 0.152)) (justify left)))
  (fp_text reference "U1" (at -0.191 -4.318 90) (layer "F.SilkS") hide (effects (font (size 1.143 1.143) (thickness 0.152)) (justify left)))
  (fp_line (start -6.604 -3.81) (end 6.396 -3.81) (width 0.254) (layer "F.SilkS") (status 40000))
  (fp_line (start 6.396 -3.81) (end 6.396 4.19) (width 0.254) (layer "F.SilkS") (status 40000))
  (fp_line (start 6.396 4.19) (end -6.604 4.19) (width 0.254) (layer "F.SilkS") (status 40000))
  (fp_line (start -6.604 4.19) (end -6.604 -3.81) (width 0.254) (layer "F.SilkS") (status 40000))
  (pad 2 thru_hole oval (at -4.445 0 90) (size 2 3.3) (layers "*.Cu" "*.Paste" "*.Mask") (drill oval 1.2 2.5) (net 5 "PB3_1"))
  (pad 1 thru_hole oval (at 0 0 90) (size 2 3.3) (layers "*.Cu" "*.Paste" "*.Mask") (drill oval 1.2 2.5) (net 15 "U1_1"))
  (pad 3 thru_hole oval (at 4.445 0 90) (size 2 3.3) (layers "*.Cu" "*.Paste" "*.Mask") (drill oval 1.2 2.5) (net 4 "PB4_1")))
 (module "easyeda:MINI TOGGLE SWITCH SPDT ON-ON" (layer "F.Cu") (at 10.08 135.382 90)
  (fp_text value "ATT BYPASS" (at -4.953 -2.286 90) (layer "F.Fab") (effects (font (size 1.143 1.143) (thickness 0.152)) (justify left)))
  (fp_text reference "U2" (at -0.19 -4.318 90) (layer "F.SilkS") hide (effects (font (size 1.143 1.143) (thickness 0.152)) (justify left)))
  (fp_line (start -6.604 -3.81) (end 6.396 -3.81) (width 0.254) (layer "F.SilkS") (status 40000))
  (fp_line (start 6.396 -3.81) (end 6.396 4.19) (width 0.254) (layer "F.SilkS") (status 40000))
  (fp_line (start 6.396 4.19) (end -6.604 4.19) (width 0.254) (layer "F.SilkS") (status 40000))
  (fp_line (start -6.604 4.19) (end -6.604 -3.81) (width 0.254) (layer "F.SilkS") (status 40000))
  (pad 2 thru_hole oval (at -4.445 0 90) (size 2 3.3) (layers "*.Cu" "*.Paste" "*.Mask") (drill oval 1.2 2.5) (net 9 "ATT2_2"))
  (pad 1 thru_hole oval (at 0 0 90) (size 2 3.3) (layers "*.Cu" "*.Paste" "*.Mask") (drill oval 1.2 2.5) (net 14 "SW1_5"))
  (pad 3 thru_hole oval (at 4.445 0 90) (size 2 3.3) (layers "*.Cu" "*.Paste" "*.Mask") (drill oval 1.2 2.5) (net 8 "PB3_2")))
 (via (at 5.691 215.295) (size 0.8) (drill 0.305) (layers "F.Cu" "B.Cu") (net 1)))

